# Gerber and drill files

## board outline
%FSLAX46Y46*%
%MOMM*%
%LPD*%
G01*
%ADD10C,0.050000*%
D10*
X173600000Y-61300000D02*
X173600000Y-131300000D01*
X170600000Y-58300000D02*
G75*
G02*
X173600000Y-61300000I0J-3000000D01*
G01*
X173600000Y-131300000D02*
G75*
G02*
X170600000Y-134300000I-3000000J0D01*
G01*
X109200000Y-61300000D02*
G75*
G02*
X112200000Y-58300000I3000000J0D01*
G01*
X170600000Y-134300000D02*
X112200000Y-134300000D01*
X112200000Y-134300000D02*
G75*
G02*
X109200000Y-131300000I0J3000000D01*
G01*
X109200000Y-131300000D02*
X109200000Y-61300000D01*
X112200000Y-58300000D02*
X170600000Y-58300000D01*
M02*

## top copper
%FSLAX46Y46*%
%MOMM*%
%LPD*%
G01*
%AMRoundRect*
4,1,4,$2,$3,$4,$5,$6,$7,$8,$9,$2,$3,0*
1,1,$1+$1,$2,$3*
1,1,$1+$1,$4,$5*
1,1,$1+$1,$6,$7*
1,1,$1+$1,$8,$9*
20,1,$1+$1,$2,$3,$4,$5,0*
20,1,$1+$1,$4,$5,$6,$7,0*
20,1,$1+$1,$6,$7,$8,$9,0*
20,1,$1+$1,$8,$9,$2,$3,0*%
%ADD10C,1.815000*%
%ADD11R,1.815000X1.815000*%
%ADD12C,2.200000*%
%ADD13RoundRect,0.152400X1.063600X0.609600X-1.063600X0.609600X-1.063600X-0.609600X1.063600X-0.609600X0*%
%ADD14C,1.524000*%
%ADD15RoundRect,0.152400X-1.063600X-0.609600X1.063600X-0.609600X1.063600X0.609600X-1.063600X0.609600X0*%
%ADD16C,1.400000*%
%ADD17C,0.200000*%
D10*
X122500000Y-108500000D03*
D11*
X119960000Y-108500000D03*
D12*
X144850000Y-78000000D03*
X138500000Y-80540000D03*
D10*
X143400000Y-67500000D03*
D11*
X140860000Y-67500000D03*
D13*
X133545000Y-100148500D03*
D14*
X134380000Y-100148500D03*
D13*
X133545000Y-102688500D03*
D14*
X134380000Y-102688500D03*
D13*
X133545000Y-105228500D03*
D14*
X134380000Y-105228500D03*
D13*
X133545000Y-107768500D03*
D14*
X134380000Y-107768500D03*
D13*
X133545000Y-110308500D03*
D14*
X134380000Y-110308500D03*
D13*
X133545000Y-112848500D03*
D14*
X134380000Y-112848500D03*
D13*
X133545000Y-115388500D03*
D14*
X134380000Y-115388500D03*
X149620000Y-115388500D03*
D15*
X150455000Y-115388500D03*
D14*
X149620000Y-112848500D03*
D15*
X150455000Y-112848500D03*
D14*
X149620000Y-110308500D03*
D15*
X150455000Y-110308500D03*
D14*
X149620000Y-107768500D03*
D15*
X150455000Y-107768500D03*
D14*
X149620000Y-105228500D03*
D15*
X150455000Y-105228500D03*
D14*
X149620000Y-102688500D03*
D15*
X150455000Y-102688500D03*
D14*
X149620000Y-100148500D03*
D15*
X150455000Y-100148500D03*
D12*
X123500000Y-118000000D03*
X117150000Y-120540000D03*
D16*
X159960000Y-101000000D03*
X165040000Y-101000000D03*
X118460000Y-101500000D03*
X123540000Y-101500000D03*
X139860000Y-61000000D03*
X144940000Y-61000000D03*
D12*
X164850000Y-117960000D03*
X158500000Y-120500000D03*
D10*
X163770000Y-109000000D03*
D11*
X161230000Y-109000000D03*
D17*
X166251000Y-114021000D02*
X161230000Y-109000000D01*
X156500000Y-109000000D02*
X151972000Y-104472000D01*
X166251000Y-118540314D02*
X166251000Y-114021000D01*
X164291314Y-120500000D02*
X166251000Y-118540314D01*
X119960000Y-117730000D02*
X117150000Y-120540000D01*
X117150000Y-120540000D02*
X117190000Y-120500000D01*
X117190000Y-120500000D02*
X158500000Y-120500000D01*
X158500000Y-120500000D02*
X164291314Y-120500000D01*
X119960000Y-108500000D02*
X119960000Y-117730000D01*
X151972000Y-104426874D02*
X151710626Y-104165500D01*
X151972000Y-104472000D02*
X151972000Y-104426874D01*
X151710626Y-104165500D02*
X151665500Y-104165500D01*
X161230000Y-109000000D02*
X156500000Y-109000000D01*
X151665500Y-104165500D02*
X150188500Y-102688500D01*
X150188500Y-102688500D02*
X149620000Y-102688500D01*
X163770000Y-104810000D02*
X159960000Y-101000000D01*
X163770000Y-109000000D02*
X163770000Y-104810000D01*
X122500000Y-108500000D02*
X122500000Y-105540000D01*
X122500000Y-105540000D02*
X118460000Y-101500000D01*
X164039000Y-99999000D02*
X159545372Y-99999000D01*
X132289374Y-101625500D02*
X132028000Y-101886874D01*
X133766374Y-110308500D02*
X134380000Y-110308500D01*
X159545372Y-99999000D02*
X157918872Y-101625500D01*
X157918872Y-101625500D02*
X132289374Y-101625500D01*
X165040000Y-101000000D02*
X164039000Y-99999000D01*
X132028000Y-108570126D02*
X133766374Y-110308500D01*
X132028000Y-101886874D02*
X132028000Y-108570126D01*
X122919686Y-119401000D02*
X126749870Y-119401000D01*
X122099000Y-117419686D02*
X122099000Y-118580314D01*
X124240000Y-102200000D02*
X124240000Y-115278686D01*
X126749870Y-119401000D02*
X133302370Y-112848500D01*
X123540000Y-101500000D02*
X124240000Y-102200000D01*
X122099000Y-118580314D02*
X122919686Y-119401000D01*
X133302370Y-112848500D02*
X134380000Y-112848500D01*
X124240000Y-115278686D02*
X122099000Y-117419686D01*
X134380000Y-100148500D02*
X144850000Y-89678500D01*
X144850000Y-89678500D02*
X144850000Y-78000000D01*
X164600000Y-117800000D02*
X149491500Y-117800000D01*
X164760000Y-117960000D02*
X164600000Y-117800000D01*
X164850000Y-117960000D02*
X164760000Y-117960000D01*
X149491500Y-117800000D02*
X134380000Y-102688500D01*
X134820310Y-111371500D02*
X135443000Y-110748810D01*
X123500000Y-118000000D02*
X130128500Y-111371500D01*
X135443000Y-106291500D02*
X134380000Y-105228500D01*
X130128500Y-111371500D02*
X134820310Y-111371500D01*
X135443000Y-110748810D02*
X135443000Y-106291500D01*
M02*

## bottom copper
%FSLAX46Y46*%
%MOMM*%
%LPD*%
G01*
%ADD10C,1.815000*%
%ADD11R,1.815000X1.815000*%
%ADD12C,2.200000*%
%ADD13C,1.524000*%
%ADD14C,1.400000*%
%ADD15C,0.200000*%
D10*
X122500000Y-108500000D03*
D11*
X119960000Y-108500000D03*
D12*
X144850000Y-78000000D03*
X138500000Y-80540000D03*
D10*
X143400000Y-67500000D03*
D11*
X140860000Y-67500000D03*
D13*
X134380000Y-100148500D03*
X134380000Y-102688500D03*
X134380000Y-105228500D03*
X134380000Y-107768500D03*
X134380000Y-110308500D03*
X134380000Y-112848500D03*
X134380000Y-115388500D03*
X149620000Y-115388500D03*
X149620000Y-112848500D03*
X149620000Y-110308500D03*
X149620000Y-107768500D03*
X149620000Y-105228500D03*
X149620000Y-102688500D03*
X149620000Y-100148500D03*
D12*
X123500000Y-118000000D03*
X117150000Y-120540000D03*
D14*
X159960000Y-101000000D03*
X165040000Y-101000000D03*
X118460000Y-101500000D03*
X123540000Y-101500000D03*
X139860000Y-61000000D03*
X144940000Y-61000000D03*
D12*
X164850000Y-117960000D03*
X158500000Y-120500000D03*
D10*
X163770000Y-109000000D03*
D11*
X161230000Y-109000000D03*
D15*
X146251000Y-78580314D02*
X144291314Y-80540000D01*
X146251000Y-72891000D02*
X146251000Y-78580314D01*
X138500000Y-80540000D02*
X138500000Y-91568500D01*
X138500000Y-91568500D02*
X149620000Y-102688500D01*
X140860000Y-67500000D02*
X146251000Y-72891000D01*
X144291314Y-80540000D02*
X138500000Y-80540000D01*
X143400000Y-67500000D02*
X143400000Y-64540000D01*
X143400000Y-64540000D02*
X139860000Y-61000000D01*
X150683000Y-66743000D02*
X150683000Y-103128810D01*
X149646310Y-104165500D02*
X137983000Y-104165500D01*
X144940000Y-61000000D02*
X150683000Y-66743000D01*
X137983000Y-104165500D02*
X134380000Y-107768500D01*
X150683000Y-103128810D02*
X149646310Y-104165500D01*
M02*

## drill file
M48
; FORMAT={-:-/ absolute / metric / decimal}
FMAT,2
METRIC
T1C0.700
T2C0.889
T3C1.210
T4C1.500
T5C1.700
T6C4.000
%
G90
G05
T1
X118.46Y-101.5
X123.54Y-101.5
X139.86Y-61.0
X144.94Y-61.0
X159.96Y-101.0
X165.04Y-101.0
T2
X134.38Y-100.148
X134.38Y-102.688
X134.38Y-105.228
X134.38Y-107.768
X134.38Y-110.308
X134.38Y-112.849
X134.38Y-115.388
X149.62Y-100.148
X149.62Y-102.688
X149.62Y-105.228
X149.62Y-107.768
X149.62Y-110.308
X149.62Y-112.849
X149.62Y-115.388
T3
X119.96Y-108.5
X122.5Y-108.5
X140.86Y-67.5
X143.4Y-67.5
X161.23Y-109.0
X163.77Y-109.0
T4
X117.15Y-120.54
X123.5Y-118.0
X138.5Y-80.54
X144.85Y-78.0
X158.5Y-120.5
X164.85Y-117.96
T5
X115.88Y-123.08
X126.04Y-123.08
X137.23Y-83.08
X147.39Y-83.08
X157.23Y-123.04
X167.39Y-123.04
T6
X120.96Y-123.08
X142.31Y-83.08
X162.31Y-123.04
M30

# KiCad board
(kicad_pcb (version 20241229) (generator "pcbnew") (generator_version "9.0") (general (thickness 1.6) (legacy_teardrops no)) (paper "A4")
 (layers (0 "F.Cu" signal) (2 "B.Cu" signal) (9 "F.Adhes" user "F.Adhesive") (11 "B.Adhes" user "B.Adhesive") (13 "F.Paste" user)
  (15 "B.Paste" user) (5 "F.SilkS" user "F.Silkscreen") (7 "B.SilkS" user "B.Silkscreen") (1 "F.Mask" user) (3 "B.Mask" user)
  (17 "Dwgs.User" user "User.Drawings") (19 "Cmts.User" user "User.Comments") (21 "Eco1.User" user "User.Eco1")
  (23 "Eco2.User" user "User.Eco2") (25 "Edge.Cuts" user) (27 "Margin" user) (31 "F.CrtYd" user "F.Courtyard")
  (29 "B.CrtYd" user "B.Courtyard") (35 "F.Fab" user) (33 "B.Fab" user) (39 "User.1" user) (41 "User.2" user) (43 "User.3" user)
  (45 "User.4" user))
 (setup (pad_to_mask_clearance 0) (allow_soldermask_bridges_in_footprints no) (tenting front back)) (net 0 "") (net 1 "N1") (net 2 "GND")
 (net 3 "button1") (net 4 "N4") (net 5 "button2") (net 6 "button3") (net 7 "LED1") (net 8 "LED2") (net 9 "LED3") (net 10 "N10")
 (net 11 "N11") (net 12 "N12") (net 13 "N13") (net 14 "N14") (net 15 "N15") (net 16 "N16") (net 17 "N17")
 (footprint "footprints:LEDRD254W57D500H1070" (layer "F.Cu") (at 121.23 108.5)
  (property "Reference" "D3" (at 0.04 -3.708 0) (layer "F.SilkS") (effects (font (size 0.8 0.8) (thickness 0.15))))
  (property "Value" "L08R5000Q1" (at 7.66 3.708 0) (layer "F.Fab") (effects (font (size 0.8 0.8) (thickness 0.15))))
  (pad "A" thru_hole circle (at 1.27 0) (size 1.815 1.815) (drill 1.21) (layers "*.Cu" "*.Mask") (remove_unused_layers no) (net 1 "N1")
   (solder_mask_margin 0.102))
  (pad "C" thru_hole rect (at -1.27 0) (size 1.815 1.815) (drill 1.21) (layers "*.Cu" "*.Mask") (remove_unused_layers no) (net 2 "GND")
   (solder_mask_margin 0.102)))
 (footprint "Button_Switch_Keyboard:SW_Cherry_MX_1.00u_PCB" (layer "F.Cu") (at 144.85 78)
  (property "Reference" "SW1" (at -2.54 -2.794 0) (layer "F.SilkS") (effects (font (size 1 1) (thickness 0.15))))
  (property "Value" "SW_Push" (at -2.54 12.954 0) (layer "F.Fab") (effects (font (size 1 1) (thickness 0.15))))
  (pad "" np_thru_hole circle (at -7.62 5.08) (size 1.7 1.7) (drill 1.7) (layers "*.Cu" "*.Mask"))
  (pad "" np_thru_hole circle (at -2.54 5.08) (size 4 4) (drill 4) (layers "*.Cu" "*.Mask"))
  (pad "" np_thru_hole circle (at 2.54 5.08) (size 1.7 1.7) (drill 1.7) (layers "*.Cu" "*.Mask"))
  (pad "1" thru_hole circle (at 0 0) (size 2.2 2.2) (drill 1.5) (layers "*.Cu" "*.Mask") (remove_unused_layers no) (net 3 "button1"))
  (pad "2" thru_hole circle (at -6.35 2.54) (size 2.2 2.2) (drill 1.5) (layers "*.Cu" "*.Mask") (remove_unused_layers no) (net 2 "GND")))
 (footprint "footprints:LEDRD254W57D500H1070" (layer "F.Cu") (at 142.13 67.5)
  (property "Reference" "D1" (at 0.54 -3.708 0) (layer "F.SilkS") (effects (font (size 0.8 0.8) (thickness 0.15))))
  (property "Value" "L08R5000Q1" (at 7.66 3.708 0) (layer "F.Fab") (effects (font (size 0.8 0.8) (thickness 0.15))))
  (pad "A" thru_hole circle (at 1.27 0) (size 1.815 1.815) (drill 1.21) (layers "*.Cu" "*.Mask") (remove_unused_layers no) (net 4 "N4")
   (solder_mask_margin 0.102))
  (pad "C" thru_hole rect (at -1.27 0) (size 1.815 1.815) (drill 1.21) (layers "*.Cu" "*.Mask") (remove_unused_layers no) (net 2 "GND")
   (solder_mask_margin 0.102)))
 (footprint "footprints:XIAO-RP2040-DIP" (layer "F.Cu") (at 142 107.7685)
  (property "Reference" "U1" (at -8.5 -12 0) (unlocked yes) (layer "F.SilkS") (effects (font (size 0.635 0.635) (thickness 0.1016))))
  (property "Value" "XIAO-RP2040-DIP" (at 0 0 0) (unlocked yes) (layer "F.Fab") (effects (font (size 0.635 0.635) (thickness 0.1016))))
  (pad "1" smd roundrect (at -8.455 -7.62 180) (size 2.432 1.524) (layers "F.Cu" "F.Mask") (roundrect_rratio 0.1) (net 3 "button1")
   (thermal_bridge_angle 45))
  (pad "1" thru_hole circle (at -7.62 -7.62 180) (size 1.524 1.524) (drill 0.889) (layers "*.Cu" "*.Mask") (remove_unused_layers no)
   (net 3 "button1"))
  (pad "2" smd roundrect (at -8.455 -5.08 180) (size 2.432 1.524) (layers "F.Cu" "F.Mask") (roundrect_rratio 0.1) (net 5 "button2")
   (thermal_bridge_angle 45))
  (pad "2" thru_hole circle (at -7.62 -5.08 180) (size 1.524 1.524) (drill 0.889) (layers "*.Cu" "*.Mask") (remove_unused_layers no)
   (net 5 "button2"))
  (pad "3" smd roundrect (at -8.455 -2.54 180) (size 2.432 1.524) (layers "F.Cu" "F.Mask") (roundrect_rratio 0.1) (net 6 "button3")
   (thermal_bridge_angle 45))
  (pad "3" thru_hole circle (at -7.62 -2.54 180) (size 1.524 1.524) (drill 0.889) (layers "*.Cu" "*.Mask") (remove_unused_layers no)
   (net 6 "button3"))
  (pad "4" smd roundrect (at -8.455 0 180) (size 2.432 1.524) (layers "F.Cu" "F.Mask") (roundrect_rratio 0.1) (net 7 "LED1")
   (thermal_bridge_angle 45))
  (pad "4" thru_hole circle (at -7.62 0 180) (size 1.524 1.524) (drill 0.889) (layers "*.Cu" "*.Mask") (remove_unused_layers no)
   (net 7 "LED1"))
  (pad "5" smd roundrect (at -8.455 2.54 180) (size 2.432 1.524) (layers "F.Cu" "F.Mask") (roundrect_rratio 0.1) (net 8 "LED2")
   (thermal_bridge_angle 45))
  (pad "5" thru_hole circle (at -7.62 2.54 180) (size 1.524 1.524) (drill 0.889) (layers "*.Cu" "*.Mask") (remove_unused_layers no)
   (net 8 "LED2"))
  (pad "6" smd roundrect (at -8.455 5.08 180) (size 2.432 1.524) (layers "F.Cu" "F.Mask") (roundrect_rratio 0.1) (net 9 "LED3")
   (thermal_bridge_angle 45))
  (pad "6" thru_hole circle (at -7.62 5.08 180) (size 1.524 1.524) (drill 0.889) (layers "*.Cu" "*.Mask") (remove_unused_layers no)
   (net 9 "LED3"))
  (pad "7" smd roundrect (at -8.455 7.62 180) (size 2.432 1.524) (layers "F.Cu" "F.Mask") (roundrect_rratio 0.1) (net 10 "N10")
   (thermal_bridge_angle 45))
  (pad "7" thru_hole circle (at -7.62 7.62 180) (size 1.524 1.524) (drill 0.889) (layers "*.Cu" "*.Mask") (remove_unused_layers no)
   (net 10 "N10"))
  (pad "8" thru_hole circle (at 7.62 7.62) (size 1.524 1.524) (drill 0.889) (layers "*.Cu" "*.Mask") (remove_unused_layers no)
   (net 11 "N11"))
  (pad "8" smd roundrect (at 8.455 7.62) (size 2.432 1.524) (layers "F.Cu" "F.Mask") (roundrect_rratio 0.1) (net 11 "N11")
   (thermal_bridge_angle 45))
  (pad "9" thru_hole circle (at 7.62 5.08) (size 1.524 1.524) (drill 0.889) (layers "*.Cu" "*.Mask") (remove_unused_layers no)
   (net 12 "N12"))
  (pad "9" smd roundrect (at 8.455 5.08) (size 2.432 1.524) (layers "F.Cu" "F.Mask") (roundrect_rratio 0.1) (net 12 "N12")
   (thermal_bridge_angle 45))
  (pad "10" thru_hole circle (at 7.62 2.54) (size 1.524 1.524) (drill 0.889) (layers "*.Cu" "*.Mask") (remove_unused_layers no)
   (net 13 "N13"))
  (pad "10" smd roundrect (at 8.455 2.54) (size 2.432 1.524) (layers "F.Cu" "F.Mask") (roundrect_rratio 0.1) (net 13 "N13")
   (thermal_bridge_angle 45))
  (pad "11" thru_hole circle (at 7.62 0) (size 1.524 1.524) (drill 0.889) (layers "*.Cu" "*.Mask") (remove_unused_layers no) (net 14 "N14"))
  (pad "11" smd roundrect (at 8.455 0) (size 2.432 1.524) (layers "F.Cu" "F.Mask") (roundrect_rratio 0.1) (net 14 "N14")
   (thermal_bridge_angle 45))
  (pad "12" thru_hole circle (at 7.62 -2.54) (size 1.524 1.524) (drill 0.889) (layers "*.Cu" "*.Mask") (remove_unused_layers no)
   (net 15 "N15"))
  (pad "12" smd roundrect (at 8.455 -2.54) (size 2.432 1.524) (layers "F.Cu" "F.Mask") (roundrect_rratio 0.1) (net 15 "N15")
   (thermal_bridge_angle 45))
  (pad "13" thru_hole circle (at 7.62 -5.08) (size 1.524 1.524) (drill 0.889) (layers "*.Cu" "*.Mask") (remove_unused_layers no)
   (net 2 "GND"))
  (pad "13" smd roundrect (at 8.455 -5.08) (size 2.432 1.524) (layers "F.Cu" "F.Mask") (roundrect_rratio 0.1) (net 2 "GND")
   (thermal_bridge_angle 45))
  (pad "14" thru_hole circle (at 7.62 -7.62) (size 1.524 1.524) (drill 0.889) (layers "*.Cu" "*.Mask") (remove_unused_layers no)
   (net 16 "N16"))
  (pad "14" smd roundrect (at 8.455 -7.62) (size 2.432 1.524) (layers "F.Cu" "F.Mask") (roundrect_rratio 0.1) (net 16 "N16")
   (thermal_bridge_angle 45)))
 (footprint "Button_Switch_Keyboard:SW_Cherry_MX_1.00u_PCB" (layer "F.Cu") (at 123.5 118)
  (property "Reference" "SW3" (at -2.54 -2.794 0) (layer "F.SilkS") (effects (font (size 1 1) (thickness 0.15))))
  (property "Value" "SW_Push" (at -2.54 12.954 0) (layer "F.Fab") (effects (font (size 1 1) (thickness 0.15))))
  (pad "" np_thru_hole circle (at -7.62 5.08) (size 1.7 1.7) (drill 1.7) (layers "*.Cu" "*.Mask"))
  (pad "" np_thru_hole circle (at -2.54 5.08) (size 4 4) (drill 4) (layers "*.Cu" "*.Mask"))
  (pad "" np_thru_hole circle (at 2.54 5.08) (size 1.7 1.7) (drill 1.7) (layers "*.Cu" "*.Mask"))
  (pad "1" thru_hole circle (at 0 0) (size 2.2 2.2) (drill 1.5) (layers "*.Cu" "*.Mask") (remove_unused_layers no) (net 6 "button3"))
  (pad "2" thru_hole circle (at -6.35 2.54) (size 2.2 2.2) (drill 1.5) (layers "*.Cu" "*.Mask") (remove_unused_layers no) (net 2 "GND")))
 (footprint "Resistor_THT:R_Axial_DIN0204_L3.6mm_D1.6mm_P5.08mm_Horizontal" (layer "F.Cu") (at 159.96 101)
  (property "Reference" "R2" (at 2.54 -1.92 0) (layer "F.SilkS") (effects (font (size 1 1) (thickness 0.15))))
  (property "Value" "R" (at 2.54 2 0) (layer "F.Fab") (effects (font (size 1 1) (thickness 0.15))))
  (pad "1" thru_hole circle (at 0 0) (size 1.4 1.4) (drill 0.7) (layers "*.Cu" "*.Mask") (remove_unused_layers no) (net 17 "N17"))
  (pad "2" thru_hole circle (at 5.08 0) (size 1.4 1.4) (drill 0.7) (layers "*.Cu" "*.Mask") (remove_unused_layers no) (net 8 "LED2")))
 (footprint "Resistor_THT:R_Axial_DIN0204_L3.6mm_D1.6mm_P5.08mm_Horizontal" (layer "F.Cu") (at 118.46 101.5)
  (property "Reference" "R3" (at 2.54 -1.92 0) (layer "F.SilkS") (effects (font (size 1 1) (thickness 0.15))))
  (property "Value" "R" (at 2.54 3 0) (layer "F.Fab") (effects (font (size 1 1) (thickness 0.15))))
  (pad "1" thru_hole circle (at 0 0) (size 1.4 1.4) (drill 0.7) (layers "*.Cu" "*.Mask") (remove_unused_layers no) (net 1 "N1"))
  (pad "2" thru_hole circle (at 5.08 0) (size 1.4 1.4) (drill 0.7) (layers "*.Cu" "*.Mask") (remove_unused_layers no) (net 9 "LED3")))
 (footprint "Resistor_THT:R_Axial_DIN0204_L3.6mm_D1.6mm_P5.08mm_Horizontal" (layer "F.Cu") (at 139.86 61)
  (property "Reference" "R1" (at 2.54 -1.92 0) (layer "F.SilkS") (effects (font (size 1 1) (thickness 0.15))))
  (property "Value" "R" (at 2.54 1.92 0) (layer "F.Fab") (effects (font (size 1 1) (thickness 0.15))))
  (pad "1" thru_hole circle (at 0 0) (size 1.4 1.4) (drill 0.7) (layers "*.Cu" "*.Mask") (remove_unused_layers no) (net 4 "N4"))
  (pad "2" thru_hole circle (at 5.08 0) (size 1.4 1.4) (drill 0.7) (layers "*.Cu" "*.Mask") (remove_unused_layers no) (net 7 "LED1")))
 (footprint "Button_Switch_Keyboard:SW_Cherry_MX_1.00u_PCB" (layer "F.Cu") (at 164.85 117.96)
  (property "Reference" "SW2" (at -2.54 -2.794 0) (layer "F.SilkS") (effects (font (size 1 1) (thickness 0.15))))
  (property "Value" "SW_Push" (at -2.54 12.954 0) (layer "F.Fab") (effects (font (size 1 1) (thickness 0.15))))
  (pad "" np_thru_hole circle (at -7.62 5.08) (size 1.7 1.7) (drill 1.7) (layers "*.Cu" "*.Mask"))
  (pad "" np_thru_hole circle (at -2.54 5.08) (size 4 4) (drill 4) (layers "*.Cu" "*.Mask"))
  (pad "" np_thru_hole circle (at 2.54 5.08) (size 1.7 1.7) (drill 1.7) (layers "*.Cu" "*.Mask"))
  (pad "1" thru_hole circle (at 0 0) (size 2.2 2.2) (drill 1.5) (layers "*.Cu" "*.Mask") (remove_unused_layers no) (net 5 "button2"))
  (pad "2" thru_hole circle (at -6.35 2.54) (size 2.2 2.2) (drill 1.5) (layers "*.Cu" "*.Mask") (remove_unused_layers no) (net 2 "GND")))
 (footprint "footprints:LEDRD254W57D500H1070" (layer "F.Cu") (at 162.5 109)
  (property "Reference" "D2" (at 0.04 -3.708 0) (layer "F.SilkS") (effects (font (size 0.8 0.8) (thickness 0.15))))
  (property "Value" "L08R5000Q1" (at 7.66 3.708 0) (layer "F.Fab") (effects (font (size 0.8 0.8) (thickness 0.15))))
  (pad "A" thru_hole circle (at 1.27 0) (size 1.815 1.815) (drill 1.21) (layers "*.Cu" "*.Mask") (remove_unused_layers no) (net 17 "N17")
   (solder_mask_margin 0.102))
  (pad "C" thru_hole rect (at -1.27 0) (size 1.815 1.815) (drill 1.21) (layers "*.Cu" "*.Mask") (remove_unused_layers no) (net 2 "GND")
   (solder_mask_margin 0.102)))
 (gr_line (start 173.6 61.3) (end 173.6 131.3) (stroke (width 0.05) (type default)) (layer "Edge.Cuts"))
 (gr_arc (start 170.6 58.3) (mid 172.72132 59.17868) (end 173.6 61.3) (stroke (width 0.05) (type default)) (layer "Edge.Cuts"))
 (gr_arc (start 173.6 131.3) (mid 172.72132 133.42132) (end 170.6 134.3) (stroke (width 0.05) (type default)) (layer "Edge.Cuts"))
 (gr_arc (start 109.2 61.3) (mid 110.07868 59.17868) (end 112.2 58.3) (stroke (width 0.05) (type default)) (layer "Edge.Cuts"))
 (gr_line (start 170.6 134.3) (end 112.2 134.3) (stroke (width 0.05) (type default)) (layer "Edge.Cuts"))
 (gr_arc (start 112.2 134.3) (mid 110.07868 133.42132) (end 109.2 131.3) (stroke (width 0.05) (type default)) (layer "Edge.Cuts"))
 (gr_line (start 109.2 131.3) (end 109.2 61.3) (stroke (width 0.05) (type default)) (layer "Edge.Cuts"))
 (gr_line (start 112.2 58.3) (end 170.6 58.3) (stroke (width 0.05) (type default)) (layer "Edge.Cuts"))
 (segment (start 166.251 114.021) (end 161.23 109) (width 0.2) (layer "F.Cu") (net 2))
 (segment (start 156.5 109) (end 151.972 104.472) (width 0.2) (layer "F.Cu") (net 2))
 (segment (start 166.251 118.540314) (end 166.251 114.021) (width 0.2) (layer "F.Cu") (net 2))
 (segment (start 164.291314 120.5) (end 166.251 118.540314) (width 0.2) (layer "F.Cu") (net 2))
 (segment (start 119.96 117.73) (end 117.15 120.54) (width 0.2) (layer "F.Cu") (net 2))
 (segment (start 117.15 120.54) (end 117.19 120.5) (width 0.2) (layer "F.Cu") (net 2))
 (segment (start 117.19 120.5) (end 158.5 120.5) (width 0.2) (layer "F.Cu") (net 2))
 (segment (start 158.5 120.5) (end 164.291314 120.5) (width 0.2) (layer "F.Cu") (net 2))
 (segment (start 119.96 108.5) (end 119.96 117.73) (width 0.2) (layer "F.Cu") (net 2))
 (segment (start 151.972 104.426874) (end 151.710626 104.1655) (width 0.2) (layer "F.Cu") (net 2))
 (segment (start 151.972 104.472) (end 151.972 104.426874) (width 0.2) (layer "F.Cu") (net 2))
 (segment (start 151.710626 104.1655) (end 151.6655 104.1655) (width 0.2) (layer "F.Cu") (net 2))
 (segment (start 161.23 109) (end 156.5 109) (width 0.2) (layer "F.Cu") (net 2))
 (segment (start 151.6655 104.1655) (end 150.1885 102.6885) (width 0.2) (layer "F.Cu") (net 2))
 (segment (start 150.1885 102.6885) (end 149.62 102.6885) (width 0.2) (layer "F.Cu") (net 2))
 (segment (start 146.251 78.580314) (end 144.291314 80.54) (width 0.2) (layer "B.Cu") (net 2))
 (segment (start 146.251 72.891) (end 146.251 78.580314) (width 0.2) (layer "B.Cu") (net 2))
 (segment (start 138.5 80.54) (end 138.5 91.5685) (width 0.2) (layer "B.Cu") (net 2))
 (segment (start 138.5 91.5685) (end 149.62 102.6885) (width 0.2) (layer "B.Cu") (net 2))
 (segment (start 140.86 67.5) (end 146.251 72.891) (width 0.2) (layer "B.Cu") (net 2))
 (segment (start 144.291314 80.54) (end 138.5 80.54) (width 0.2) (layer "B.Cu") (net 2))
 (segment (start 143.4 67.5) (end 143.4 64.54) (width 0.2) (layer "B.Cu") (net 4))
 (segment (start 143.4 64.54) (end 139.86 61) (width 0.2) (layer "B.Cu") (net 4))
 (segment (start 163.77 104.81) (end 159.96 101) (width 0.2) (layer "F.Cu") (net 17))
 (segment (start 163.77 109) (end 163.77 104.81) (width 0.2) (layer "F.Cu") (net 17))
 (segment (start 122.5 108.5) (end 122.5 105.54) (width 0.2) (layer "F.Cu") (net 1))
 (segment (start 122.5 105.54) (end 118.46 101.5) (width 0.2) (layer "F.Cu") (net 1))
 (segment (start 150.683 66.743) (end 150.683 103.12881) (width 0.2) (layer "B.Cu") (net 7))
 (segment (start 149.64631 104.1655) (end 137.983 104.1655) (width 0.2) (layer "B.Cu") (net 7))
 (segment (start 144.94 61) (end 150.683 66.743) (width 0.2) (layer "B.Cu") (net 7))
 (segment (start 137.983 104.1655) (end 134.38 107.7685) (width 0.2) (layer "B.Cu") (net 7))
 (segment (start 150.683 103.12881) (end 149.64631 104.1655) (width 0.2) (layer "B.Cu") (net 7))
 (segment (start 164.039 99.999) (end 159.545372 99.999) (width 0.2) (layer "F.Cu") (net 8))
 (segment (start 132.289374 101.6255) (end 132.028 101.886874) (width 0.2) (layer "F.Cu") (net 8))
 (segment (start 133.766374 110.3085) (end 134.38 110.3085) (width 0.2) (layer "F.Cu") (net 8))
 (segment (start 159.545372 99.999) (end 157.918872 101.6255) (width 0.2) (layer "F.Cu") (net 8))
 (segment (start 157.918872 101.6255) (end 132.289374 101.6255) (width 0.2) (layer "F.Cu") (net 8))
 (segment (start 165.04 101) (end 164.039 99.999) (width 0.2) (layer "F.Cu") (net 8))
 (segment (start 132.028 108.570126) (end 133.766374 110.3085) (width 0.2) (layer "F.Cu") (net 8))
 (segment (start 132.028 101.886874) (end 132.028 108.570126) (width 0.2) (layer "F.Cu") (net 8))
 (segment (start 122.919686 119.401) (end 126.74987 119.401) (width 0.2) (layer "F.Cu") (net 9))
 (segment (start 122.099 117.419686) (end 122.099 118.580314) (width 0.2) (layer "F.Cu") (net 9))
 (segment (start 124.24 102.2) (end 124.24 115.278686) (width 0.2) (layer "F.Cu") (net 9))
 (segment (start 126.74987 119.401) (end 133.30237 112.8485) (width 0.2) (layer "F.Cu") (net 9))
 (segment (start 123.54 101.5) (end 124.24 102.2) (width 0.2) (layer "F.Cu") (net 9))
 (segment (start 122.099 118.580314) (end 122.919686 119.401) (width 0.2) (layer "F.Cu") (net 9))
 (segment (start 133.30237 112.8485) (end 134.38 112.8485) (width 0.2) (layer "F.Cu") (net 9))
 (segment (start 124.24 115.278686) (end 122.099 117.419686) (width 0.2) (layer "F.Cu") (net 9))
 (segment (start 134.38 100.1485) (end 144.85 89.6785) (width 0.2) (layer "F.Cu") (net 3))
 (segment (start 144.85 89.6785) (end 144.85 78) (width 0.2) (layer "F.Cu") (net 3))
 (segment (start 164.6 117.8) (end 149.4915 117.8) (width 0.2) (layer "F.Cu") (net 5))
 (segment (start 164.76 117.96) (end 164.6 117.8) (width 0.2) (layer "F.Cu") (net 5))
 (segment (start 164.85 117.96) (end 164.76 117.96) (width 0.2) (layer "F.Cu") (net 5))
 (segment (start 149.4915 117.8) (end 134.38 102.6885) (width 0.2) (layer "F.Cu") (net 5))
 (segment (start 134.82031 111.3715) (end 135.443 110.74881) (width 0.2) (layer "F.Cu") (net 6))
 (segment (start 123.5 118) (end 130.1285 111.3715) (width 0.2) (layer "F.Cu") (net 6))
 (segment (start 135.443 106.2915) (end 134.38 105.2285) (width 0.2) (layer "F.Cu") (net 6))
 (segment (start 130.1285 111.3715) (end 134.82031 111.3715) (width 0.2) (layer "F.Cu") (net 6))
 (segment (start 135.443 110.74881) (end 135.443 106.2915) (width 0.2) (layer "F.Cu") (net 6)))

